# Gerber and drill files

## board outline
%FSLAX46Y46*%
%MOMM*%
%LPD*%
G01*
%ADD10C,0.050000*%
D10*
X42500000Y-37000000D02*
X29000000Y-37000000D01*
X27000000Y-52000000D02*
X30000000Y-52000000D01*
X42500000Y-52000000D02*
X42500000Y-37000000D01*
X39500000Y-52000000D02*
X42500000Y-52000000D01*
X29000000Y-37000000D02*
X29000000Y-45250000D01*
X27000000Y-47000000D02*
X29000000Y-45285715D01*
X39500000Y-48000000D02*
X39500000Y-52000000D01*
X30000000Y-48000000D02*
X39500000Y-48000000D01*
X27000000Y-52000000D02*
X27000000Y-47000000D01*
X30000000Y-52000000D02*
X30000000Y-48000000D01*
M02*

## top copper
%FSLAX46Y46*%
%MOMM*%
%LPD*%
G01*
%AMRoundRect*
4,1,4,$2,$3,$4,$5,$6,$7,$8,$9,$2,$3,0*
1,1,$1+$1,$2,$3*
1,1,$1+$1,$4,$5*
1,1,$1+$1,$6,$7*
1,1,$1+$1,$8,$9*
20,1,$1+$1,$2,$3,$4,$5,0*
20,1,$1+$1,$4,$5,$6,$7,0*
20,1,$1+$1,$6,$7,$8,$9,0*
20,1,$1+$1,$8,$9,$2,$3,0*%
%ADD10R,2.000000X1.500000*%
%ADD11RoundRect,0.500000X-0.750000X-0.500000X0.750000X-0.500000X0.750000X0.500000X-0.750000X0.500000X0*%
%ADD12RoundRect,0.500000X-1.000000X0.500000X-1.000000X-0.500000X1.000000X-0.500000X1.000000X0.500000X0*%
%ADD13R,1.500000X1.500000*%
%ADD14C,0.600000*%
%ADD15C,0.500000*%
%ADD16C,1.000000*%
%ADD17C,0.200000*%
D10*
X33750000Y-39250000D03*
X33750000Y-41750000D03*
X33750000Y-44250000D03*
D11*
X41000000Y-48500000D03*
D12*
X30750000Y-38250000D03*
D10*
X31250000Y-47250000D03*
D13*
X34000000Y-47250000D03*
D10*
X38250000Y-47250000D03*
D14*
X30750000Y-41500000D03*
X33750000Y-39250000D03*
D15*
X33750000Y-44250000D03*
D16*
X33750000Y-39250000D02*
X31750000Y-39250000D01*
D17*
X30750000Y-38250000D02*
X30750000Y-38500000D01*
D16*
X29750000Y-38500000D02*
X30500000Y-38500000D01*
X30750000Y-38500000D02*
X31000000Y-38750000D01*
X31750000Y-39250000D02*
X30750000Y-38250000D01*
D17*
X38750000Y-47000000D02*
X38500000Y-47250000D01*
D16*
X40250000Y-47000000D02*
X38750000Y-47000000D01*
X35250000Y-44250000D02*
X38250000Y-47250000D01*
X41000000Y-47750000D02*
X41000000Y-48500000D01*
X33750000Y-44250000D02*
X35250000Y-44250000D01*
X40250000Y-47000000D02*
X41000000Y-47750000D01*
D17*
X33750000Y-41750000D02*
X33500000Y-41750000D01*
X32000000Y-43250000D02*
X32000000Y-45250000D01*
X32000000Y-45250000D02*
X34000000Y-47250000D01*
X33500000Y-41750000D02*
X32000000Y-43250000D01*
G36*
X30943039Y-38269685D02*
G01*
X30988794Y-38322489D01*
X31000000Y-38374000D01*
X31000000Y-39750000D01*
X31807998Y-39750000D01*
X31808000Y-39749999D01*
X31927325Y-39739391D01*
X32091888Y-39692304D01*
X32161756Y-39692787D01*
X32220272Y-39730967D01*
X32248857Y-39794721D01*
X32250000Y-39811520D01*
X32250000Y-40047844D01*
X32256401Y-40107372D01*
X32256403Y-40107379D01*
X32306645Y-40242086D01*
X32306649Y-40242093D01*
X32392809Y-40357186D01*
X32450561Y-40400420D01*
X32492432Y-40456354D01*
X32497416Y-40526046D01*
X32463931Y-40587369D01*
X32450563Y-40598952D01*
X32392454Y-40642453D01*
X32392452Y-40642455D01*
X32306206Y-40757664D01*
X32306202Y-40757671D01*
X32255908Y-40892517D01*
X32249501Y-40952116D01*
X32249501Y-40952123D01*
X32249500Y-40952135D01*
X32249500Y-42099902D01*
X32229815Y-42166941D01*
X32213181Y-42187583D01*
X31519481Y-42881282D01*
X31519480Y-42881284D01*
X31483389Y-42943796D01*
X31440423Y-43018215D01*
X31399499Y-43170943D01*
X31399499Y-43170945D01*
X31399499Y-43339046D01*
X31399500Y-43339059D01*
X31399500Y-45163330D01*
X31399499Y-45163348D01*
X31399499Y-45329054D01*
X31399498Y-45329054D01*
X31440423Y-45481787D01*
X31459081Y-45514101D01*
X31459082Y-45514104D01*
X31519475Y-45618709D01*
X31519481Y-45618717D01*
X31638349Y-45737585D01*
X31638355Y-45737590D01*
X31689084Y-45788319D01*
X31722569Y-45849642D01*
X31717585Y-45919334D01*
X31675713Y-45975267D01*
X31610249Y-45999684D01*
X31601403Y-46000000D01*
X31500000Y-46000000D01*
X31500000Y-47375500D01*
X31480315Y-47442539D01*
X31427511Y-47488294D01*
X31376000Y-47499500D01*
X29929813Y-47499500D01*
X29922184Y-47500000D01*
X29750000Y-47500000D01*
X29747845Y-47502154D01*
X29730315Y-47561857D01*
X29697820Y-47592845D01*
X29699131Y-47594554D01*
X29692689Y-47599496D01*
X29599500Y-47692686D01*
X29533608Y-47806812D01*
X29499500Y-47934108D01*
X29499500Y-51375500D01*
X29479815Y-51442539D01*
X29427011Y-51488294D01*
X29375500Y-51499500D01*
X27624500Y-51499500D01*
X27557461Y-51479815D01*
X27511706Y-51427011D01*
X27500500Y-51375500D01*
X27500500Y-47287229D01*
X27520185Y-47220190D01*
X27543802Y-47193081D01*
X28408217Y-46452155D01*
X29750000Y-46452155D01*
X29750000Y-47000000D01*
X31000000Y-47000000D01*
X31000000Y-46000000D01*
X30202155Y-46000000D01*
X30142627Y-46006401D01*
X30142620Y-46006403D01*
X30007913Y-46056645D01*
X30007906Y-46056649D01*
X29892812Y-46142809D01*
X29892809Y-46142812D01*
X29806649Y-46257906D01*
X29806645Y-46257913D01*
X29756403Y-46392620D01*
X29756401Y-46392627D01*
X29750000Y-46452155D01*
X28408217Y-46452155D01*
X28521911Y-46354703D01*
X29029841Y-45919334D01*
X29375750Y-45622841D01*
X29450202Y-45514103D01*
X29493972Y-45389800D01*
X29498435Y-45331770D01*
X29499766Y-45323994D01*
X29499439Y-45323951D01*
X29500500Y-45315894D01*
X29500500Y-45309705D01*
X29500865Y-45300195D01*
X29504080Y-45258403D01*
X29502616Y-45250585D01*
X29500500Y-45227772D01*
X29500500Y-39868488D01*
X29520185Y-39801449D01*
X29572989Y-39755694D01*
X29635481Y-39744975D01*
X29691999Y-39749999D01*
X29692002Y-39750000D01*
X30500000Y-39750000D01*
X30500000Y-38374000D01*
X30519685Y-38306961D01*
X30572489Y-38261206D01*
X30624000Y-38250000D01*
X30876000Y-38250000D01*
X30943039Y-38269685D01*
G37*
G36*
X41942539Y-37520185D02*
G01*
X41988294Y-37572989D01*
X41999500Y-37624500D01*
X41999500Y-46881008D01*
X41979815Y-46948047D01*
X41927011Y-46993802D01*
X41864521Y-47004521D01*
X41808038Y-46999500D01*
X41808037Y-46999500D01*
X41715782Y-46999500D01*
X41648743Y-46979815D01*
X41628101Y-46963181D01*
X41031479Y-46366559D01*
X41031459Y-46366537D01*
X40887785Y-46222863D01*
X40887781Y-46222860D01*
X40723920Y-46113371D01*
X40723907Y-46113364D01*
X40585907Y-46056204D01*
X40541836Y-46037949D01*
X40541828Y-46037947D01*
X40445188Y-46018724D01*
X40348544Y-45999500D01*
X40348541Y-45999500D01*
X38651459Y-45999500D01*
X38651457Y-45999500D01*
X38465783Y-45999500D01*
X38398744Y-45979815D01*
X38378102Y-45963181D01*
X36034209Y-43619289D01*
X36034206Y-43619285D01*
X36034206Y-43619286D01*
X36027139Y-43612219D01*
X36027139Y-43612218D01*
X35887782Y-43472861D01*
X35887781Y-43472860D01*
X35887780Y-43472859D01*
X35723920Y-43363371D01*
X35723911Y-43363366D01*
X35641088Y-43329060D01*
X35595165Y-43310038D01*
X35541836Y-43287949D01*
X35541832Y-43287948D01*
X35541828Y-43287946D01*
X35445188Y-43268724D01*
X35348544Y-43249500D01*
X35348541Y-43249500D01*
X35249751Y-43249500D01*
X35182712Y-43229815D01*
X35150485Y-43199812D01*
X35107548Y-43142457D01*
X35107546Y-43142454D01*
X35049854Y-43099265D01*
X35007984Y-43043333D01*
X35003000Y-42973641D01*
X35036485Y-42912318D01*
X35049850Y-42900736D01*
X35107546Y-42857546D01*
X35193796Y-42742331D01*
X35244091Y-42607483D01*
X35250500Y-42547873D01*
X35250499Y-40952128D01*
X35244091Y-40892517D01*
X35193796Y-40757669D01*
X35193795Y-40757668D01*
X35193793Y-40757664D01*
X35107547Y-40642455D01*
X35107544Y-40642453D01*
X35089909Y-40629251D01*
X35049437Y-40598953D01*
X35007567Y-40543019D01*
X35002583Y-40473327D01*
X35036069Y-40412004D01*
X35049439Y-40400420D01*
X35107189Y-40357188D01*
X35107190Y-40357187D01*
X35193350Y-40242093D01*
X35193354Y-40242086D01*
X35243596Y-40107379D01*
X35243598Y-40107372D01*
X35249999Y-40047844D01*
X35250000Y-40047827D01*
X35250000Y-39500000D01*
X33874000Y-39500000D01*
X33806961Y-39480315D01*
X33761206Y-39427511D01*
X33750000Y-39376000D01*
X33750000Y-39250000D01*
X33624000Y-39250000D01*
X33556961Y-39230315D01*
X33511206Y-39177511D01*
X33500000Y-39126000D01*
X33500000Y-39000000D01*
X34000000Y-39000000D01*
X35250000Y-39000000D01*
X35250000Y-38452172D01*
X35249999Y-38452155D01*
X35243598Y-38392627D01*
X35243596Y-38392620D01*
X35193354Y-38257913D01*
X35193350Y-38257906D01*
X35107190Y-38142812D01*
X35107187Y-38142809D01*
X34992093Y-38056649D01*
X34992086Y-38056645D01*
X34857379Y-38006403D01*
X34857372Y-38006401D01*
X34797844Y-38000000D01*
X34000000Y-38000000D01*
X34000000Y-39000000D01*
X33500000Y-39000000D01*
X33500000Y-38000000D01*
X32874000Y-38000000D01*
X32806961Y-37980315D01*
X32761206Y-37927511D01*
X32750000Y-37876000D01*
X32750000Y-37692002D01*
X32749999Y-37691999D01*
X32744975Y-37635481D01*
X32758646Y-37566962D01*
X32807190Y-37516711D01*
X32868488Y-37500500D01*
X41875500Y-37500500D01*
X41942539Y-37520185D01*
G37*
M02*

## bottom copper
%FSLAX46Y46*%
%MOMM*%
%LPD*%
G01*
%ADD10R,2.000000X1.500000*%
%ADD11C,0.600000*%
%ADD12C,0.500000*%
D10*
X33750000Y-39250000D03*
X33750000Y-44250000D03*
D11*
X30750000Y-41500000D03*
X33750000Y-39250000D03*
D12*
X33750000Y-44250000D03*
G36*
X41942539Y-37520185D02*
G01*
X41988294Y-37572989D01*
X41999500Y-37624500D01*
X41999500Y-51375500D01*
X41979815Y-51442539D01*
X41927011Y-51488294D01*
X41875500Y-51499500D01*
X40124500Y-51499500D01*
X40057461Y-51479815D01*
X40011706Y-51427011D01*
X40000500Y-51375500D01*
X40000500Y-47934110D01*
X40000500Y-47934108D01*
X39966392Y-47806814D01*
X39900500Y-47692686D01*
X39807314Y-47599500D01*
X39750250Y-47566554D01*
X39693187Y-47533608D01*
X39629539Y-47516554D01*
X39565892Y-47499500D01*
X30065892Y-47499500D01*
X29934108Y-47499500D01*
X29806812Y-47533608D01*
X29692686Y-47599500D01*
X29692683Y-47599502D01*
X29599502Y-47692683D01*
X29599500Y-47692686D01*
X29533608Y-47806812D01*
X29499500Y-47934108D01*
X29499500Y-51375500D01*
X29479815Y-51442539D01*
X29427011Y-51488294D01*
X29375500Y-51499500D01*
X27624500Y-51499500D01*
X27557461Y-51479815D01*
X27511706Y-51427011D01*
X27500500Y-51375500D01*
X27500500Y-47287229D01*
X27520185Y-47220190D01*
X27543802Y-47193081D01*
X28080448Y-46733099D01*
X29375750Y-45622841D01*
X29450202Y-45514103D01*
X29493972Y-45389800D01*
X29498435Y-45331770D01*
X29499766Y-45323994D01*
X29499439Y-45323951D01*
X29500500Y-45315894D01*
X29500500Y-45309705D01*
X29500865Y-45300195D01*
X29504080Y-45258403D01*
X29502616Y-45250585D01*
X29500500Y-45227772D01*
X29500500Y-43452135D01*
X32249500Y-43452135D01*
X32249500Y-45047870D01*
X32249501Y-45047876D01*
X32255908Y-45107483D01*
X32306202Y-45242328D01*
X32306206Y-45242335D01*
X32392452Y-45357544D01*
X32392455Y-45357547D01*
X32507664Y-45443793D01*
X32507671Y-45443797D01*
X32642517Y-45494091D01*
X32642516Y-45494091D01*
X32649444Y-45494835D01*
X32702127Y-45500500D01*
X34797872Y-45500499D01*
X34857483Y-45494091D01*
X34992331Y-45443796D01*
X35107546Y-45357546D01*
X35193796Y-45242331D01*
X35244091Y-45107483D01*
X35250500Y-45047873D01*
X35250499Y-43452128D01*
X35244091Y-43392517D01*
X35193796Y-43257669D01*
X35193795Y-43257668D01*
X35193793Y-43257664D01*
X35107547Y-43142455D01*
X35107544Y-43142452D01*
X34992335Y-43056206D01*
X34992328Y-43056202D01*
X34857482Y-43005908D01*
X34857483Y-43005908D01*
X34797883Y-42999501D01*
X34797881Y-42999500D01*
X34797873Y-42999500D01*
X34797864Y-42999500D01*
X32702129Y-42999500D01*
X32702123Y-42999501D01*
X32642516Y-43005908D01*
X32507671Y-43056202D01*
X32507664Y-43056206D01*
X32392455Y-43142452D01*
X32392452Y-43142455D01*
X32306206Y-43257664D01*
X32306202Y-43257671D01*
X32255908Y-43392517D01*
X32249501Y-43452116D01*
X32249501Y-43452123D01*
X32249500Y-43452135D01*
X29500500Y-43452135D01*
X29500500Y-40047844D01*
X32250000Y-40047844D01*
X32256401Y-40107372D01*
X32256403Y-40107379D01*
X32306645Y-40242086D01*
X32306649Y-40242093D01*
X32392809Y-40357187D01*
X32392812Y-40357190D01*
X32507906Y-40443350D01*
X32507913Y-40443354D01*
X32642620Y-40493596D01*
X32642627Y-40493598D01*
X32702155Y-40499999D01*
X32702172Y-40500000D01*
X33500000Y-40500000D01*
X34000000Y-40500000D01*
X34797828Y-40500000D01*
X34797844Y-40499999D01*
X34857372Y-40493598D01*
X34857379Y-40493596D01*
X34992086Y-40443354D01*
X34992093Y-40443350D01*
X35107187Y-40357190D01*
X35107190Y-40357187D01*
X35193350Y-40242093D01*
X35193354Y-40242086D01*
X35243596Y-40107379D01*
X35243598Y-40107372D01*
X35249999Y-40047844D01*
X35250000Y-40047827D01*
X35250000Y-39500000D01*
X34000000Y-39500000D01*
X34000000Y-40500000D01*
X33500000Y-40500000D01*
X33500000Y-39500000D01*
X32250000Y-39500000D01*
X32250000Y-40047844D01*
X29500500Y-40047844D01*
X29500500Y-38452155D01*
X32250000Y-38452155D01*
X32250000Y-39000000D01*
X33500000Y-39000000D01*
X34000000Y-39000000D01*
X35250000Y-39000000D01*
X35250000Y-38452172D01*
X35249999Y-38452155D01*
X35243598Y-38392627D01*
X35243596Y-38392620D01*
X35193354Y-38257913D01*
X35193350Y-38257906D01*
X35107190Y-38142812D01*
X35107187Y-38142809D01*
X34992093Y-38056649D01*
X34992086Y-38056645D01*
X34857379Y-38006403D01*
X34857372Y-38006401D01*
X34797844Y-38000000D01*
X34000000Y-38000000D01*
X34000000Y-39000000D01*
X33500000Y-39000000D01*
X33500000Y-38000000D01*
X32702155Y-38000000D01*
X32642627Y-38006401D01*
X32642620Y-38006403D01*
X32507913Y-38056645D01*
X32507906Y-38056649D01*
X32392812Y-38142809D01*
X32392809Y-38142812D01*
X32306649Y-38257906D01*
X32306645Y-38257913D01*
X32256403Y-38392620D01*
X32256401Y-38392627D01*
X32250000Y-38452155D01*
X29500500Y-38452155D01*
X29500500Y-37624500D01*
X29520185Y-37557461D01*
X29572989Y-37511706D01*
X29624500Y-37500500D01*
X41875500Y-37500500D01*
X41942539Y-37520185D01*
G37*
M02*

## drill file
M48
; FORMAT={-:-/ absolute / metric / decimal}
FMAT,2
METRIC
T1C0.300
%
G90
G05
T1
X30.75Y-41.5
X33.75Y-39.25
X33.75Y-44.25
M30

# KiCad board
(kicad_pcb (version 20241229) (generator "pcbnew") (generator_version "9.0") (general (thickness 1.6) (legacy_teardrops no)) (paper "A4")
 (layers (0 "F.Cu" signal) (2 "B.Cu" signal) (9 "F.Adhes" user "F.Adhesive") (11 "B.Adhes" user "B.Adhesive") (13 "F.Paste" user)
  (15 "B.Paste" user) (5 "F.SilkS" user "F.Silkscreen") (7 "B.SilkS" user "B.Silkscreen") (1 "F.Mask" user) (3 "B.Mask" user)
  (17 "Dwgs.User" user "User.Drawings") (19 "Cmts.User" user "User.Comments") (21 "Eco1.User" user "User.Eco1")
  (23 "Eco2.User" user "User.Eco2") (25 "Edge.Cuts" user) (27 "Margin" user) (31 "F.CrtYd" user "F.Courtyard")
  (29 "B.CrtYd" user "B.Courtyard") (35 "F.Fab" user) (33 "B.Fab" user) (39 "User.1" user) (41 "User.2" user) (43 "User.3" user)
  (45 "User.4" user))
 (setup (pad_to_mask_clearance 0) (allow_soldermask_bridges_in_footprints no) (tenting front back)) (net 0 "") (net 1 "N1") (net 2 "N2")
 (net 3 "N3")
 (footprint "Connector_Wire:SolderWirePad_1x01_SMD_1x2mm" (layer "F.Cu") (at 33.75 44.25)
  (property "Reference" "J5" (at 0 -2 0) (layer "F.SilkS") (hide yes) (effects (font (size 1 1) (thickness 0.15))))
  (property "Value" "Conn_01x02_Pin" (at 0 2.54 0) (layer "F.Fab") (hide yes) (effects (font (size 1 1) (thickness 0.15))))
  (pad "1" smd rect (at 0 -5 270) (size 1.5 2) (layers "B.Cu" "B.Mask") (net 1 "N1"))
  (pad "2" smd rect (at 0 0 270) (size 1.5 2) (layers "B.Cu" "B.Mask") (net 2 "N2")))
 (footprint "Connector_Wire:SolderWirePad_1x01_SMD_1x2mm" (layer "F.Cu") (at 33.75 43)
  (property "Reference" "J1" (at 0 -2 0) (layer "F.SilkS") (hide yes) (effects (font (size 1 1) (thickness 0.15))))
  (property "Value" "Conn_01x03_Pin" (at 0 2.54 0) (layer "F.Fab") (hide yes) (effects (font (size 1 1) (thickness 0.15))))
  (pad "1" smd rect (at 0 -3.75 90) (size 1.5 2) (layers "F.Cu" "F.Mask" "F.Paste") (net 1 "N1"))
  (pad "2" smd rect (at 0 -1.25 90) (size 1.5 2) (layers "F.Cu" "F.Mask") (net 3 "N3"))
  (pad "3" smd rect (at 0 1.25 90) (size 1.5 2) (layers "F.Cu" "F.Mask") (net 2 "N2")))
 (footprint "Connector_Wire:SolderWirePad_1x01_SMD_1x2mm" (layer "F.Cu") (at 41.25 48.5)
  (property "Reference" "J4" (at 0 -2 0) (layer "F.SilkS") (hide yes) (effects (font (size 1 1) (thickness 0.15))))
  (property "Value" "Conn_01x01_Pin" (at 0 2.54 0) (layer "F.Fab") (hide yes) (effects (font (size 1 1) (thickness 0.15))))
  (pad "1" smd roundrect (at -0.25 0) (size 2.5 2) (layers "F.Cu" "F.Mask") (roundrect_rratio 0.25) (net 2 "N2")))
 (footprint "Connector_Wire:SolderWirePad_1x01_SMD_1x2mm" (layer "F.Cu") (at 30.75 38.25 -90)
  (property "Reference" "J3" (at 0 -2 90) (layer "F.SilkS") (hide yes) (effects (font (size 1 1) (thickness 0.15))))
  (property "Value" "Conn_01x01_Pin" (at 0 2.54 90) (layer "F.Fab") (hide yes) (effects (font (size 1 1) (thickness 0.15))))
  (pad "1" smd roundrect (at 0 0 270) (size 2 3) (layers "F.Cu" "F.Mask") (roundrect_rratio 0.25) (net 1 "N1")))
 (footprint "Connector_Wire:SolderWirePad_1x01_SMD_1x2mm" (layer "F.Cu") (at 30 47)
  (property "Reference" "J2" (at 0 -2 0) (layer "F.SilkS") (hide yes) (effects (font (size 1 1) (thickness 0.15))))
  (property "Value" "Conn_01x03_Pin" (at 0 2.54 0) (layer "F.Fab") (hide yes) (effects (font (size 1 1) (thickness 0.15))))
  (pad "1" smd rect (at 1.25 0.25) (size 2 1.5) (layers "F.Cu" "F.Mask") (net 1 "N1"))
  (pad "2" smd rect (at 4 0.25) (size 1.5 1.5) (layers "F.Cu" "F.Mask") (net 3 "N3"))
  (pad "3" smd rect (at 8.25 0.25) (size 2 1.5) (layers "F.Cu" "F.Mask") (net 2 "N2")))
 (gr_line (start 42.5 37) (end 29 37) (stroke (width 0.05) (type default)) (layer "Edge.Cuts"))
 (gr_line (start 27 52) (end 30 52) (stroke (width 0.05) (type default)) (layer "Edge.Cuts"))
 (gr_line (start 42.5 52) (end 42.5 37) (stroke (width 0.05) (type default)) (layer "Edge.Cuts"))
 (gr_line (start 39.5 52) (end 42.5 52) (stroke (width 0.05) (type default)) (layer "Edge.Cuts"))
 (gr_line (start 29 37) (end 29 45.25) (stroke (width 0.05) (type default)) (layer "Edge.Cuts"))
 (gr_line (start 27 47) (end 29 45.285715) (stroke (width 0.05) (type default)) (layer "Edge.Cuts"))
 (gr_line (start 39.5 48) (end 39.5 52) (stroke (width 0.05) (type default)) (layer "Edge.Cuts"))
 (gr_line (start 30 48) (end 39.5 48) (stroke (width 0.05) (type default)) (layer "Edge.Cuts"))
 (gr_line (start 27 52) (end 27 47) (stroke (width 0.05) (type default)) (layer "Edge.Cuts"))
 (gr_line (start 30 52) (end 30 48) (stroke (width 0.05) (type default)) (layer "Edge.Cuts"))
 (segment (start 33.75 39.25) (end 31.75 39.25) (width 1) (layer "F.Cu") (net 1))
 (segment (start 30.75 38.25) (end 30.75 38.5) (width 0.2) (layer "F.Cu") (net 1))
 (segment (start 29.75 38.5) (end 30.5 38.5) (width 1) (layer "F.Cu") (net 1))
 (segment (start 30.75 38.5) (end 31 38.75) (width 1) (layer "F.Cu") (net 1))
 (segment (start 31.75 39.25) (end 30.75 38.25) (width 1) (layer "F.Cu") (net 1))
 (via (at 30.75 41.5) (size 0.6) (drill 0.3) (layers "F.Cu" "B.Cu") (free yes) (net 1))
 (via (at 33.75 39.25) (size 0.6) (drill 0.3) (layers "F.Cu" "B.Cu") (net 1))
 (segment (start 38.75 47) (end 38.5 47.25) (width 0.2) (layer "F.Cu") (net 2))
 (segment (start 40.25 47) (end 38.75 47) (width 1) (layer "F.Cu") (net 2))
 (segment (start 35.25 44.25) (end 38.25 47.25) (width 1) (layer "F.Cu") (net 2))
 (segment (start 41 47.75) (end 41 48.5) (width 1) (layer "F.Cu") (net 2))
 (segment (start 33.75 44.25) (end 35.25 44.25) (width 1) (layer "F.Cu") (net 2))
 (segment (start 40.25 47) (end 41 47.75) (width 1) (layer "F.Cu") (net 2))
 (via (at 33.75 44.25) (size 0.5) (drill 0.3) (layers "F.Cu" "B.Cu") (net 2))
 (segment (start 33.75 41.75) (end 33.5 41.75) (width 0.2) (layer "F.Cu") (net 3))
 (segment (start 32 43.25) (end 32 45.25) (width 0.2) (layer "F.Cu") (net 3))
 (segment (start 32 45.25) (end 34 47.25) (width 0.2) (layer "F.Cu") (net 3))
 (segment (start 33.5 41.75) (end 32 43.25) (width 0.2) (layer "F.Cu") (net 3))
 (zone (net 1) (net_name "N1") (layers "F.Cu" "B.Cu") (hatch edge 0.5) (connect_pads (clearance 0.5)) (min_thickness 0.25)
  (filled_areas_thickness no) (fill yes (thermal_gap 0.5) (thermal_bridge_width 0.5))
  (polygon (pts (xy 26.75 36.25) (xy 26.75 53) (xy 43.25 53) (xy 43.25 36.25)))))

